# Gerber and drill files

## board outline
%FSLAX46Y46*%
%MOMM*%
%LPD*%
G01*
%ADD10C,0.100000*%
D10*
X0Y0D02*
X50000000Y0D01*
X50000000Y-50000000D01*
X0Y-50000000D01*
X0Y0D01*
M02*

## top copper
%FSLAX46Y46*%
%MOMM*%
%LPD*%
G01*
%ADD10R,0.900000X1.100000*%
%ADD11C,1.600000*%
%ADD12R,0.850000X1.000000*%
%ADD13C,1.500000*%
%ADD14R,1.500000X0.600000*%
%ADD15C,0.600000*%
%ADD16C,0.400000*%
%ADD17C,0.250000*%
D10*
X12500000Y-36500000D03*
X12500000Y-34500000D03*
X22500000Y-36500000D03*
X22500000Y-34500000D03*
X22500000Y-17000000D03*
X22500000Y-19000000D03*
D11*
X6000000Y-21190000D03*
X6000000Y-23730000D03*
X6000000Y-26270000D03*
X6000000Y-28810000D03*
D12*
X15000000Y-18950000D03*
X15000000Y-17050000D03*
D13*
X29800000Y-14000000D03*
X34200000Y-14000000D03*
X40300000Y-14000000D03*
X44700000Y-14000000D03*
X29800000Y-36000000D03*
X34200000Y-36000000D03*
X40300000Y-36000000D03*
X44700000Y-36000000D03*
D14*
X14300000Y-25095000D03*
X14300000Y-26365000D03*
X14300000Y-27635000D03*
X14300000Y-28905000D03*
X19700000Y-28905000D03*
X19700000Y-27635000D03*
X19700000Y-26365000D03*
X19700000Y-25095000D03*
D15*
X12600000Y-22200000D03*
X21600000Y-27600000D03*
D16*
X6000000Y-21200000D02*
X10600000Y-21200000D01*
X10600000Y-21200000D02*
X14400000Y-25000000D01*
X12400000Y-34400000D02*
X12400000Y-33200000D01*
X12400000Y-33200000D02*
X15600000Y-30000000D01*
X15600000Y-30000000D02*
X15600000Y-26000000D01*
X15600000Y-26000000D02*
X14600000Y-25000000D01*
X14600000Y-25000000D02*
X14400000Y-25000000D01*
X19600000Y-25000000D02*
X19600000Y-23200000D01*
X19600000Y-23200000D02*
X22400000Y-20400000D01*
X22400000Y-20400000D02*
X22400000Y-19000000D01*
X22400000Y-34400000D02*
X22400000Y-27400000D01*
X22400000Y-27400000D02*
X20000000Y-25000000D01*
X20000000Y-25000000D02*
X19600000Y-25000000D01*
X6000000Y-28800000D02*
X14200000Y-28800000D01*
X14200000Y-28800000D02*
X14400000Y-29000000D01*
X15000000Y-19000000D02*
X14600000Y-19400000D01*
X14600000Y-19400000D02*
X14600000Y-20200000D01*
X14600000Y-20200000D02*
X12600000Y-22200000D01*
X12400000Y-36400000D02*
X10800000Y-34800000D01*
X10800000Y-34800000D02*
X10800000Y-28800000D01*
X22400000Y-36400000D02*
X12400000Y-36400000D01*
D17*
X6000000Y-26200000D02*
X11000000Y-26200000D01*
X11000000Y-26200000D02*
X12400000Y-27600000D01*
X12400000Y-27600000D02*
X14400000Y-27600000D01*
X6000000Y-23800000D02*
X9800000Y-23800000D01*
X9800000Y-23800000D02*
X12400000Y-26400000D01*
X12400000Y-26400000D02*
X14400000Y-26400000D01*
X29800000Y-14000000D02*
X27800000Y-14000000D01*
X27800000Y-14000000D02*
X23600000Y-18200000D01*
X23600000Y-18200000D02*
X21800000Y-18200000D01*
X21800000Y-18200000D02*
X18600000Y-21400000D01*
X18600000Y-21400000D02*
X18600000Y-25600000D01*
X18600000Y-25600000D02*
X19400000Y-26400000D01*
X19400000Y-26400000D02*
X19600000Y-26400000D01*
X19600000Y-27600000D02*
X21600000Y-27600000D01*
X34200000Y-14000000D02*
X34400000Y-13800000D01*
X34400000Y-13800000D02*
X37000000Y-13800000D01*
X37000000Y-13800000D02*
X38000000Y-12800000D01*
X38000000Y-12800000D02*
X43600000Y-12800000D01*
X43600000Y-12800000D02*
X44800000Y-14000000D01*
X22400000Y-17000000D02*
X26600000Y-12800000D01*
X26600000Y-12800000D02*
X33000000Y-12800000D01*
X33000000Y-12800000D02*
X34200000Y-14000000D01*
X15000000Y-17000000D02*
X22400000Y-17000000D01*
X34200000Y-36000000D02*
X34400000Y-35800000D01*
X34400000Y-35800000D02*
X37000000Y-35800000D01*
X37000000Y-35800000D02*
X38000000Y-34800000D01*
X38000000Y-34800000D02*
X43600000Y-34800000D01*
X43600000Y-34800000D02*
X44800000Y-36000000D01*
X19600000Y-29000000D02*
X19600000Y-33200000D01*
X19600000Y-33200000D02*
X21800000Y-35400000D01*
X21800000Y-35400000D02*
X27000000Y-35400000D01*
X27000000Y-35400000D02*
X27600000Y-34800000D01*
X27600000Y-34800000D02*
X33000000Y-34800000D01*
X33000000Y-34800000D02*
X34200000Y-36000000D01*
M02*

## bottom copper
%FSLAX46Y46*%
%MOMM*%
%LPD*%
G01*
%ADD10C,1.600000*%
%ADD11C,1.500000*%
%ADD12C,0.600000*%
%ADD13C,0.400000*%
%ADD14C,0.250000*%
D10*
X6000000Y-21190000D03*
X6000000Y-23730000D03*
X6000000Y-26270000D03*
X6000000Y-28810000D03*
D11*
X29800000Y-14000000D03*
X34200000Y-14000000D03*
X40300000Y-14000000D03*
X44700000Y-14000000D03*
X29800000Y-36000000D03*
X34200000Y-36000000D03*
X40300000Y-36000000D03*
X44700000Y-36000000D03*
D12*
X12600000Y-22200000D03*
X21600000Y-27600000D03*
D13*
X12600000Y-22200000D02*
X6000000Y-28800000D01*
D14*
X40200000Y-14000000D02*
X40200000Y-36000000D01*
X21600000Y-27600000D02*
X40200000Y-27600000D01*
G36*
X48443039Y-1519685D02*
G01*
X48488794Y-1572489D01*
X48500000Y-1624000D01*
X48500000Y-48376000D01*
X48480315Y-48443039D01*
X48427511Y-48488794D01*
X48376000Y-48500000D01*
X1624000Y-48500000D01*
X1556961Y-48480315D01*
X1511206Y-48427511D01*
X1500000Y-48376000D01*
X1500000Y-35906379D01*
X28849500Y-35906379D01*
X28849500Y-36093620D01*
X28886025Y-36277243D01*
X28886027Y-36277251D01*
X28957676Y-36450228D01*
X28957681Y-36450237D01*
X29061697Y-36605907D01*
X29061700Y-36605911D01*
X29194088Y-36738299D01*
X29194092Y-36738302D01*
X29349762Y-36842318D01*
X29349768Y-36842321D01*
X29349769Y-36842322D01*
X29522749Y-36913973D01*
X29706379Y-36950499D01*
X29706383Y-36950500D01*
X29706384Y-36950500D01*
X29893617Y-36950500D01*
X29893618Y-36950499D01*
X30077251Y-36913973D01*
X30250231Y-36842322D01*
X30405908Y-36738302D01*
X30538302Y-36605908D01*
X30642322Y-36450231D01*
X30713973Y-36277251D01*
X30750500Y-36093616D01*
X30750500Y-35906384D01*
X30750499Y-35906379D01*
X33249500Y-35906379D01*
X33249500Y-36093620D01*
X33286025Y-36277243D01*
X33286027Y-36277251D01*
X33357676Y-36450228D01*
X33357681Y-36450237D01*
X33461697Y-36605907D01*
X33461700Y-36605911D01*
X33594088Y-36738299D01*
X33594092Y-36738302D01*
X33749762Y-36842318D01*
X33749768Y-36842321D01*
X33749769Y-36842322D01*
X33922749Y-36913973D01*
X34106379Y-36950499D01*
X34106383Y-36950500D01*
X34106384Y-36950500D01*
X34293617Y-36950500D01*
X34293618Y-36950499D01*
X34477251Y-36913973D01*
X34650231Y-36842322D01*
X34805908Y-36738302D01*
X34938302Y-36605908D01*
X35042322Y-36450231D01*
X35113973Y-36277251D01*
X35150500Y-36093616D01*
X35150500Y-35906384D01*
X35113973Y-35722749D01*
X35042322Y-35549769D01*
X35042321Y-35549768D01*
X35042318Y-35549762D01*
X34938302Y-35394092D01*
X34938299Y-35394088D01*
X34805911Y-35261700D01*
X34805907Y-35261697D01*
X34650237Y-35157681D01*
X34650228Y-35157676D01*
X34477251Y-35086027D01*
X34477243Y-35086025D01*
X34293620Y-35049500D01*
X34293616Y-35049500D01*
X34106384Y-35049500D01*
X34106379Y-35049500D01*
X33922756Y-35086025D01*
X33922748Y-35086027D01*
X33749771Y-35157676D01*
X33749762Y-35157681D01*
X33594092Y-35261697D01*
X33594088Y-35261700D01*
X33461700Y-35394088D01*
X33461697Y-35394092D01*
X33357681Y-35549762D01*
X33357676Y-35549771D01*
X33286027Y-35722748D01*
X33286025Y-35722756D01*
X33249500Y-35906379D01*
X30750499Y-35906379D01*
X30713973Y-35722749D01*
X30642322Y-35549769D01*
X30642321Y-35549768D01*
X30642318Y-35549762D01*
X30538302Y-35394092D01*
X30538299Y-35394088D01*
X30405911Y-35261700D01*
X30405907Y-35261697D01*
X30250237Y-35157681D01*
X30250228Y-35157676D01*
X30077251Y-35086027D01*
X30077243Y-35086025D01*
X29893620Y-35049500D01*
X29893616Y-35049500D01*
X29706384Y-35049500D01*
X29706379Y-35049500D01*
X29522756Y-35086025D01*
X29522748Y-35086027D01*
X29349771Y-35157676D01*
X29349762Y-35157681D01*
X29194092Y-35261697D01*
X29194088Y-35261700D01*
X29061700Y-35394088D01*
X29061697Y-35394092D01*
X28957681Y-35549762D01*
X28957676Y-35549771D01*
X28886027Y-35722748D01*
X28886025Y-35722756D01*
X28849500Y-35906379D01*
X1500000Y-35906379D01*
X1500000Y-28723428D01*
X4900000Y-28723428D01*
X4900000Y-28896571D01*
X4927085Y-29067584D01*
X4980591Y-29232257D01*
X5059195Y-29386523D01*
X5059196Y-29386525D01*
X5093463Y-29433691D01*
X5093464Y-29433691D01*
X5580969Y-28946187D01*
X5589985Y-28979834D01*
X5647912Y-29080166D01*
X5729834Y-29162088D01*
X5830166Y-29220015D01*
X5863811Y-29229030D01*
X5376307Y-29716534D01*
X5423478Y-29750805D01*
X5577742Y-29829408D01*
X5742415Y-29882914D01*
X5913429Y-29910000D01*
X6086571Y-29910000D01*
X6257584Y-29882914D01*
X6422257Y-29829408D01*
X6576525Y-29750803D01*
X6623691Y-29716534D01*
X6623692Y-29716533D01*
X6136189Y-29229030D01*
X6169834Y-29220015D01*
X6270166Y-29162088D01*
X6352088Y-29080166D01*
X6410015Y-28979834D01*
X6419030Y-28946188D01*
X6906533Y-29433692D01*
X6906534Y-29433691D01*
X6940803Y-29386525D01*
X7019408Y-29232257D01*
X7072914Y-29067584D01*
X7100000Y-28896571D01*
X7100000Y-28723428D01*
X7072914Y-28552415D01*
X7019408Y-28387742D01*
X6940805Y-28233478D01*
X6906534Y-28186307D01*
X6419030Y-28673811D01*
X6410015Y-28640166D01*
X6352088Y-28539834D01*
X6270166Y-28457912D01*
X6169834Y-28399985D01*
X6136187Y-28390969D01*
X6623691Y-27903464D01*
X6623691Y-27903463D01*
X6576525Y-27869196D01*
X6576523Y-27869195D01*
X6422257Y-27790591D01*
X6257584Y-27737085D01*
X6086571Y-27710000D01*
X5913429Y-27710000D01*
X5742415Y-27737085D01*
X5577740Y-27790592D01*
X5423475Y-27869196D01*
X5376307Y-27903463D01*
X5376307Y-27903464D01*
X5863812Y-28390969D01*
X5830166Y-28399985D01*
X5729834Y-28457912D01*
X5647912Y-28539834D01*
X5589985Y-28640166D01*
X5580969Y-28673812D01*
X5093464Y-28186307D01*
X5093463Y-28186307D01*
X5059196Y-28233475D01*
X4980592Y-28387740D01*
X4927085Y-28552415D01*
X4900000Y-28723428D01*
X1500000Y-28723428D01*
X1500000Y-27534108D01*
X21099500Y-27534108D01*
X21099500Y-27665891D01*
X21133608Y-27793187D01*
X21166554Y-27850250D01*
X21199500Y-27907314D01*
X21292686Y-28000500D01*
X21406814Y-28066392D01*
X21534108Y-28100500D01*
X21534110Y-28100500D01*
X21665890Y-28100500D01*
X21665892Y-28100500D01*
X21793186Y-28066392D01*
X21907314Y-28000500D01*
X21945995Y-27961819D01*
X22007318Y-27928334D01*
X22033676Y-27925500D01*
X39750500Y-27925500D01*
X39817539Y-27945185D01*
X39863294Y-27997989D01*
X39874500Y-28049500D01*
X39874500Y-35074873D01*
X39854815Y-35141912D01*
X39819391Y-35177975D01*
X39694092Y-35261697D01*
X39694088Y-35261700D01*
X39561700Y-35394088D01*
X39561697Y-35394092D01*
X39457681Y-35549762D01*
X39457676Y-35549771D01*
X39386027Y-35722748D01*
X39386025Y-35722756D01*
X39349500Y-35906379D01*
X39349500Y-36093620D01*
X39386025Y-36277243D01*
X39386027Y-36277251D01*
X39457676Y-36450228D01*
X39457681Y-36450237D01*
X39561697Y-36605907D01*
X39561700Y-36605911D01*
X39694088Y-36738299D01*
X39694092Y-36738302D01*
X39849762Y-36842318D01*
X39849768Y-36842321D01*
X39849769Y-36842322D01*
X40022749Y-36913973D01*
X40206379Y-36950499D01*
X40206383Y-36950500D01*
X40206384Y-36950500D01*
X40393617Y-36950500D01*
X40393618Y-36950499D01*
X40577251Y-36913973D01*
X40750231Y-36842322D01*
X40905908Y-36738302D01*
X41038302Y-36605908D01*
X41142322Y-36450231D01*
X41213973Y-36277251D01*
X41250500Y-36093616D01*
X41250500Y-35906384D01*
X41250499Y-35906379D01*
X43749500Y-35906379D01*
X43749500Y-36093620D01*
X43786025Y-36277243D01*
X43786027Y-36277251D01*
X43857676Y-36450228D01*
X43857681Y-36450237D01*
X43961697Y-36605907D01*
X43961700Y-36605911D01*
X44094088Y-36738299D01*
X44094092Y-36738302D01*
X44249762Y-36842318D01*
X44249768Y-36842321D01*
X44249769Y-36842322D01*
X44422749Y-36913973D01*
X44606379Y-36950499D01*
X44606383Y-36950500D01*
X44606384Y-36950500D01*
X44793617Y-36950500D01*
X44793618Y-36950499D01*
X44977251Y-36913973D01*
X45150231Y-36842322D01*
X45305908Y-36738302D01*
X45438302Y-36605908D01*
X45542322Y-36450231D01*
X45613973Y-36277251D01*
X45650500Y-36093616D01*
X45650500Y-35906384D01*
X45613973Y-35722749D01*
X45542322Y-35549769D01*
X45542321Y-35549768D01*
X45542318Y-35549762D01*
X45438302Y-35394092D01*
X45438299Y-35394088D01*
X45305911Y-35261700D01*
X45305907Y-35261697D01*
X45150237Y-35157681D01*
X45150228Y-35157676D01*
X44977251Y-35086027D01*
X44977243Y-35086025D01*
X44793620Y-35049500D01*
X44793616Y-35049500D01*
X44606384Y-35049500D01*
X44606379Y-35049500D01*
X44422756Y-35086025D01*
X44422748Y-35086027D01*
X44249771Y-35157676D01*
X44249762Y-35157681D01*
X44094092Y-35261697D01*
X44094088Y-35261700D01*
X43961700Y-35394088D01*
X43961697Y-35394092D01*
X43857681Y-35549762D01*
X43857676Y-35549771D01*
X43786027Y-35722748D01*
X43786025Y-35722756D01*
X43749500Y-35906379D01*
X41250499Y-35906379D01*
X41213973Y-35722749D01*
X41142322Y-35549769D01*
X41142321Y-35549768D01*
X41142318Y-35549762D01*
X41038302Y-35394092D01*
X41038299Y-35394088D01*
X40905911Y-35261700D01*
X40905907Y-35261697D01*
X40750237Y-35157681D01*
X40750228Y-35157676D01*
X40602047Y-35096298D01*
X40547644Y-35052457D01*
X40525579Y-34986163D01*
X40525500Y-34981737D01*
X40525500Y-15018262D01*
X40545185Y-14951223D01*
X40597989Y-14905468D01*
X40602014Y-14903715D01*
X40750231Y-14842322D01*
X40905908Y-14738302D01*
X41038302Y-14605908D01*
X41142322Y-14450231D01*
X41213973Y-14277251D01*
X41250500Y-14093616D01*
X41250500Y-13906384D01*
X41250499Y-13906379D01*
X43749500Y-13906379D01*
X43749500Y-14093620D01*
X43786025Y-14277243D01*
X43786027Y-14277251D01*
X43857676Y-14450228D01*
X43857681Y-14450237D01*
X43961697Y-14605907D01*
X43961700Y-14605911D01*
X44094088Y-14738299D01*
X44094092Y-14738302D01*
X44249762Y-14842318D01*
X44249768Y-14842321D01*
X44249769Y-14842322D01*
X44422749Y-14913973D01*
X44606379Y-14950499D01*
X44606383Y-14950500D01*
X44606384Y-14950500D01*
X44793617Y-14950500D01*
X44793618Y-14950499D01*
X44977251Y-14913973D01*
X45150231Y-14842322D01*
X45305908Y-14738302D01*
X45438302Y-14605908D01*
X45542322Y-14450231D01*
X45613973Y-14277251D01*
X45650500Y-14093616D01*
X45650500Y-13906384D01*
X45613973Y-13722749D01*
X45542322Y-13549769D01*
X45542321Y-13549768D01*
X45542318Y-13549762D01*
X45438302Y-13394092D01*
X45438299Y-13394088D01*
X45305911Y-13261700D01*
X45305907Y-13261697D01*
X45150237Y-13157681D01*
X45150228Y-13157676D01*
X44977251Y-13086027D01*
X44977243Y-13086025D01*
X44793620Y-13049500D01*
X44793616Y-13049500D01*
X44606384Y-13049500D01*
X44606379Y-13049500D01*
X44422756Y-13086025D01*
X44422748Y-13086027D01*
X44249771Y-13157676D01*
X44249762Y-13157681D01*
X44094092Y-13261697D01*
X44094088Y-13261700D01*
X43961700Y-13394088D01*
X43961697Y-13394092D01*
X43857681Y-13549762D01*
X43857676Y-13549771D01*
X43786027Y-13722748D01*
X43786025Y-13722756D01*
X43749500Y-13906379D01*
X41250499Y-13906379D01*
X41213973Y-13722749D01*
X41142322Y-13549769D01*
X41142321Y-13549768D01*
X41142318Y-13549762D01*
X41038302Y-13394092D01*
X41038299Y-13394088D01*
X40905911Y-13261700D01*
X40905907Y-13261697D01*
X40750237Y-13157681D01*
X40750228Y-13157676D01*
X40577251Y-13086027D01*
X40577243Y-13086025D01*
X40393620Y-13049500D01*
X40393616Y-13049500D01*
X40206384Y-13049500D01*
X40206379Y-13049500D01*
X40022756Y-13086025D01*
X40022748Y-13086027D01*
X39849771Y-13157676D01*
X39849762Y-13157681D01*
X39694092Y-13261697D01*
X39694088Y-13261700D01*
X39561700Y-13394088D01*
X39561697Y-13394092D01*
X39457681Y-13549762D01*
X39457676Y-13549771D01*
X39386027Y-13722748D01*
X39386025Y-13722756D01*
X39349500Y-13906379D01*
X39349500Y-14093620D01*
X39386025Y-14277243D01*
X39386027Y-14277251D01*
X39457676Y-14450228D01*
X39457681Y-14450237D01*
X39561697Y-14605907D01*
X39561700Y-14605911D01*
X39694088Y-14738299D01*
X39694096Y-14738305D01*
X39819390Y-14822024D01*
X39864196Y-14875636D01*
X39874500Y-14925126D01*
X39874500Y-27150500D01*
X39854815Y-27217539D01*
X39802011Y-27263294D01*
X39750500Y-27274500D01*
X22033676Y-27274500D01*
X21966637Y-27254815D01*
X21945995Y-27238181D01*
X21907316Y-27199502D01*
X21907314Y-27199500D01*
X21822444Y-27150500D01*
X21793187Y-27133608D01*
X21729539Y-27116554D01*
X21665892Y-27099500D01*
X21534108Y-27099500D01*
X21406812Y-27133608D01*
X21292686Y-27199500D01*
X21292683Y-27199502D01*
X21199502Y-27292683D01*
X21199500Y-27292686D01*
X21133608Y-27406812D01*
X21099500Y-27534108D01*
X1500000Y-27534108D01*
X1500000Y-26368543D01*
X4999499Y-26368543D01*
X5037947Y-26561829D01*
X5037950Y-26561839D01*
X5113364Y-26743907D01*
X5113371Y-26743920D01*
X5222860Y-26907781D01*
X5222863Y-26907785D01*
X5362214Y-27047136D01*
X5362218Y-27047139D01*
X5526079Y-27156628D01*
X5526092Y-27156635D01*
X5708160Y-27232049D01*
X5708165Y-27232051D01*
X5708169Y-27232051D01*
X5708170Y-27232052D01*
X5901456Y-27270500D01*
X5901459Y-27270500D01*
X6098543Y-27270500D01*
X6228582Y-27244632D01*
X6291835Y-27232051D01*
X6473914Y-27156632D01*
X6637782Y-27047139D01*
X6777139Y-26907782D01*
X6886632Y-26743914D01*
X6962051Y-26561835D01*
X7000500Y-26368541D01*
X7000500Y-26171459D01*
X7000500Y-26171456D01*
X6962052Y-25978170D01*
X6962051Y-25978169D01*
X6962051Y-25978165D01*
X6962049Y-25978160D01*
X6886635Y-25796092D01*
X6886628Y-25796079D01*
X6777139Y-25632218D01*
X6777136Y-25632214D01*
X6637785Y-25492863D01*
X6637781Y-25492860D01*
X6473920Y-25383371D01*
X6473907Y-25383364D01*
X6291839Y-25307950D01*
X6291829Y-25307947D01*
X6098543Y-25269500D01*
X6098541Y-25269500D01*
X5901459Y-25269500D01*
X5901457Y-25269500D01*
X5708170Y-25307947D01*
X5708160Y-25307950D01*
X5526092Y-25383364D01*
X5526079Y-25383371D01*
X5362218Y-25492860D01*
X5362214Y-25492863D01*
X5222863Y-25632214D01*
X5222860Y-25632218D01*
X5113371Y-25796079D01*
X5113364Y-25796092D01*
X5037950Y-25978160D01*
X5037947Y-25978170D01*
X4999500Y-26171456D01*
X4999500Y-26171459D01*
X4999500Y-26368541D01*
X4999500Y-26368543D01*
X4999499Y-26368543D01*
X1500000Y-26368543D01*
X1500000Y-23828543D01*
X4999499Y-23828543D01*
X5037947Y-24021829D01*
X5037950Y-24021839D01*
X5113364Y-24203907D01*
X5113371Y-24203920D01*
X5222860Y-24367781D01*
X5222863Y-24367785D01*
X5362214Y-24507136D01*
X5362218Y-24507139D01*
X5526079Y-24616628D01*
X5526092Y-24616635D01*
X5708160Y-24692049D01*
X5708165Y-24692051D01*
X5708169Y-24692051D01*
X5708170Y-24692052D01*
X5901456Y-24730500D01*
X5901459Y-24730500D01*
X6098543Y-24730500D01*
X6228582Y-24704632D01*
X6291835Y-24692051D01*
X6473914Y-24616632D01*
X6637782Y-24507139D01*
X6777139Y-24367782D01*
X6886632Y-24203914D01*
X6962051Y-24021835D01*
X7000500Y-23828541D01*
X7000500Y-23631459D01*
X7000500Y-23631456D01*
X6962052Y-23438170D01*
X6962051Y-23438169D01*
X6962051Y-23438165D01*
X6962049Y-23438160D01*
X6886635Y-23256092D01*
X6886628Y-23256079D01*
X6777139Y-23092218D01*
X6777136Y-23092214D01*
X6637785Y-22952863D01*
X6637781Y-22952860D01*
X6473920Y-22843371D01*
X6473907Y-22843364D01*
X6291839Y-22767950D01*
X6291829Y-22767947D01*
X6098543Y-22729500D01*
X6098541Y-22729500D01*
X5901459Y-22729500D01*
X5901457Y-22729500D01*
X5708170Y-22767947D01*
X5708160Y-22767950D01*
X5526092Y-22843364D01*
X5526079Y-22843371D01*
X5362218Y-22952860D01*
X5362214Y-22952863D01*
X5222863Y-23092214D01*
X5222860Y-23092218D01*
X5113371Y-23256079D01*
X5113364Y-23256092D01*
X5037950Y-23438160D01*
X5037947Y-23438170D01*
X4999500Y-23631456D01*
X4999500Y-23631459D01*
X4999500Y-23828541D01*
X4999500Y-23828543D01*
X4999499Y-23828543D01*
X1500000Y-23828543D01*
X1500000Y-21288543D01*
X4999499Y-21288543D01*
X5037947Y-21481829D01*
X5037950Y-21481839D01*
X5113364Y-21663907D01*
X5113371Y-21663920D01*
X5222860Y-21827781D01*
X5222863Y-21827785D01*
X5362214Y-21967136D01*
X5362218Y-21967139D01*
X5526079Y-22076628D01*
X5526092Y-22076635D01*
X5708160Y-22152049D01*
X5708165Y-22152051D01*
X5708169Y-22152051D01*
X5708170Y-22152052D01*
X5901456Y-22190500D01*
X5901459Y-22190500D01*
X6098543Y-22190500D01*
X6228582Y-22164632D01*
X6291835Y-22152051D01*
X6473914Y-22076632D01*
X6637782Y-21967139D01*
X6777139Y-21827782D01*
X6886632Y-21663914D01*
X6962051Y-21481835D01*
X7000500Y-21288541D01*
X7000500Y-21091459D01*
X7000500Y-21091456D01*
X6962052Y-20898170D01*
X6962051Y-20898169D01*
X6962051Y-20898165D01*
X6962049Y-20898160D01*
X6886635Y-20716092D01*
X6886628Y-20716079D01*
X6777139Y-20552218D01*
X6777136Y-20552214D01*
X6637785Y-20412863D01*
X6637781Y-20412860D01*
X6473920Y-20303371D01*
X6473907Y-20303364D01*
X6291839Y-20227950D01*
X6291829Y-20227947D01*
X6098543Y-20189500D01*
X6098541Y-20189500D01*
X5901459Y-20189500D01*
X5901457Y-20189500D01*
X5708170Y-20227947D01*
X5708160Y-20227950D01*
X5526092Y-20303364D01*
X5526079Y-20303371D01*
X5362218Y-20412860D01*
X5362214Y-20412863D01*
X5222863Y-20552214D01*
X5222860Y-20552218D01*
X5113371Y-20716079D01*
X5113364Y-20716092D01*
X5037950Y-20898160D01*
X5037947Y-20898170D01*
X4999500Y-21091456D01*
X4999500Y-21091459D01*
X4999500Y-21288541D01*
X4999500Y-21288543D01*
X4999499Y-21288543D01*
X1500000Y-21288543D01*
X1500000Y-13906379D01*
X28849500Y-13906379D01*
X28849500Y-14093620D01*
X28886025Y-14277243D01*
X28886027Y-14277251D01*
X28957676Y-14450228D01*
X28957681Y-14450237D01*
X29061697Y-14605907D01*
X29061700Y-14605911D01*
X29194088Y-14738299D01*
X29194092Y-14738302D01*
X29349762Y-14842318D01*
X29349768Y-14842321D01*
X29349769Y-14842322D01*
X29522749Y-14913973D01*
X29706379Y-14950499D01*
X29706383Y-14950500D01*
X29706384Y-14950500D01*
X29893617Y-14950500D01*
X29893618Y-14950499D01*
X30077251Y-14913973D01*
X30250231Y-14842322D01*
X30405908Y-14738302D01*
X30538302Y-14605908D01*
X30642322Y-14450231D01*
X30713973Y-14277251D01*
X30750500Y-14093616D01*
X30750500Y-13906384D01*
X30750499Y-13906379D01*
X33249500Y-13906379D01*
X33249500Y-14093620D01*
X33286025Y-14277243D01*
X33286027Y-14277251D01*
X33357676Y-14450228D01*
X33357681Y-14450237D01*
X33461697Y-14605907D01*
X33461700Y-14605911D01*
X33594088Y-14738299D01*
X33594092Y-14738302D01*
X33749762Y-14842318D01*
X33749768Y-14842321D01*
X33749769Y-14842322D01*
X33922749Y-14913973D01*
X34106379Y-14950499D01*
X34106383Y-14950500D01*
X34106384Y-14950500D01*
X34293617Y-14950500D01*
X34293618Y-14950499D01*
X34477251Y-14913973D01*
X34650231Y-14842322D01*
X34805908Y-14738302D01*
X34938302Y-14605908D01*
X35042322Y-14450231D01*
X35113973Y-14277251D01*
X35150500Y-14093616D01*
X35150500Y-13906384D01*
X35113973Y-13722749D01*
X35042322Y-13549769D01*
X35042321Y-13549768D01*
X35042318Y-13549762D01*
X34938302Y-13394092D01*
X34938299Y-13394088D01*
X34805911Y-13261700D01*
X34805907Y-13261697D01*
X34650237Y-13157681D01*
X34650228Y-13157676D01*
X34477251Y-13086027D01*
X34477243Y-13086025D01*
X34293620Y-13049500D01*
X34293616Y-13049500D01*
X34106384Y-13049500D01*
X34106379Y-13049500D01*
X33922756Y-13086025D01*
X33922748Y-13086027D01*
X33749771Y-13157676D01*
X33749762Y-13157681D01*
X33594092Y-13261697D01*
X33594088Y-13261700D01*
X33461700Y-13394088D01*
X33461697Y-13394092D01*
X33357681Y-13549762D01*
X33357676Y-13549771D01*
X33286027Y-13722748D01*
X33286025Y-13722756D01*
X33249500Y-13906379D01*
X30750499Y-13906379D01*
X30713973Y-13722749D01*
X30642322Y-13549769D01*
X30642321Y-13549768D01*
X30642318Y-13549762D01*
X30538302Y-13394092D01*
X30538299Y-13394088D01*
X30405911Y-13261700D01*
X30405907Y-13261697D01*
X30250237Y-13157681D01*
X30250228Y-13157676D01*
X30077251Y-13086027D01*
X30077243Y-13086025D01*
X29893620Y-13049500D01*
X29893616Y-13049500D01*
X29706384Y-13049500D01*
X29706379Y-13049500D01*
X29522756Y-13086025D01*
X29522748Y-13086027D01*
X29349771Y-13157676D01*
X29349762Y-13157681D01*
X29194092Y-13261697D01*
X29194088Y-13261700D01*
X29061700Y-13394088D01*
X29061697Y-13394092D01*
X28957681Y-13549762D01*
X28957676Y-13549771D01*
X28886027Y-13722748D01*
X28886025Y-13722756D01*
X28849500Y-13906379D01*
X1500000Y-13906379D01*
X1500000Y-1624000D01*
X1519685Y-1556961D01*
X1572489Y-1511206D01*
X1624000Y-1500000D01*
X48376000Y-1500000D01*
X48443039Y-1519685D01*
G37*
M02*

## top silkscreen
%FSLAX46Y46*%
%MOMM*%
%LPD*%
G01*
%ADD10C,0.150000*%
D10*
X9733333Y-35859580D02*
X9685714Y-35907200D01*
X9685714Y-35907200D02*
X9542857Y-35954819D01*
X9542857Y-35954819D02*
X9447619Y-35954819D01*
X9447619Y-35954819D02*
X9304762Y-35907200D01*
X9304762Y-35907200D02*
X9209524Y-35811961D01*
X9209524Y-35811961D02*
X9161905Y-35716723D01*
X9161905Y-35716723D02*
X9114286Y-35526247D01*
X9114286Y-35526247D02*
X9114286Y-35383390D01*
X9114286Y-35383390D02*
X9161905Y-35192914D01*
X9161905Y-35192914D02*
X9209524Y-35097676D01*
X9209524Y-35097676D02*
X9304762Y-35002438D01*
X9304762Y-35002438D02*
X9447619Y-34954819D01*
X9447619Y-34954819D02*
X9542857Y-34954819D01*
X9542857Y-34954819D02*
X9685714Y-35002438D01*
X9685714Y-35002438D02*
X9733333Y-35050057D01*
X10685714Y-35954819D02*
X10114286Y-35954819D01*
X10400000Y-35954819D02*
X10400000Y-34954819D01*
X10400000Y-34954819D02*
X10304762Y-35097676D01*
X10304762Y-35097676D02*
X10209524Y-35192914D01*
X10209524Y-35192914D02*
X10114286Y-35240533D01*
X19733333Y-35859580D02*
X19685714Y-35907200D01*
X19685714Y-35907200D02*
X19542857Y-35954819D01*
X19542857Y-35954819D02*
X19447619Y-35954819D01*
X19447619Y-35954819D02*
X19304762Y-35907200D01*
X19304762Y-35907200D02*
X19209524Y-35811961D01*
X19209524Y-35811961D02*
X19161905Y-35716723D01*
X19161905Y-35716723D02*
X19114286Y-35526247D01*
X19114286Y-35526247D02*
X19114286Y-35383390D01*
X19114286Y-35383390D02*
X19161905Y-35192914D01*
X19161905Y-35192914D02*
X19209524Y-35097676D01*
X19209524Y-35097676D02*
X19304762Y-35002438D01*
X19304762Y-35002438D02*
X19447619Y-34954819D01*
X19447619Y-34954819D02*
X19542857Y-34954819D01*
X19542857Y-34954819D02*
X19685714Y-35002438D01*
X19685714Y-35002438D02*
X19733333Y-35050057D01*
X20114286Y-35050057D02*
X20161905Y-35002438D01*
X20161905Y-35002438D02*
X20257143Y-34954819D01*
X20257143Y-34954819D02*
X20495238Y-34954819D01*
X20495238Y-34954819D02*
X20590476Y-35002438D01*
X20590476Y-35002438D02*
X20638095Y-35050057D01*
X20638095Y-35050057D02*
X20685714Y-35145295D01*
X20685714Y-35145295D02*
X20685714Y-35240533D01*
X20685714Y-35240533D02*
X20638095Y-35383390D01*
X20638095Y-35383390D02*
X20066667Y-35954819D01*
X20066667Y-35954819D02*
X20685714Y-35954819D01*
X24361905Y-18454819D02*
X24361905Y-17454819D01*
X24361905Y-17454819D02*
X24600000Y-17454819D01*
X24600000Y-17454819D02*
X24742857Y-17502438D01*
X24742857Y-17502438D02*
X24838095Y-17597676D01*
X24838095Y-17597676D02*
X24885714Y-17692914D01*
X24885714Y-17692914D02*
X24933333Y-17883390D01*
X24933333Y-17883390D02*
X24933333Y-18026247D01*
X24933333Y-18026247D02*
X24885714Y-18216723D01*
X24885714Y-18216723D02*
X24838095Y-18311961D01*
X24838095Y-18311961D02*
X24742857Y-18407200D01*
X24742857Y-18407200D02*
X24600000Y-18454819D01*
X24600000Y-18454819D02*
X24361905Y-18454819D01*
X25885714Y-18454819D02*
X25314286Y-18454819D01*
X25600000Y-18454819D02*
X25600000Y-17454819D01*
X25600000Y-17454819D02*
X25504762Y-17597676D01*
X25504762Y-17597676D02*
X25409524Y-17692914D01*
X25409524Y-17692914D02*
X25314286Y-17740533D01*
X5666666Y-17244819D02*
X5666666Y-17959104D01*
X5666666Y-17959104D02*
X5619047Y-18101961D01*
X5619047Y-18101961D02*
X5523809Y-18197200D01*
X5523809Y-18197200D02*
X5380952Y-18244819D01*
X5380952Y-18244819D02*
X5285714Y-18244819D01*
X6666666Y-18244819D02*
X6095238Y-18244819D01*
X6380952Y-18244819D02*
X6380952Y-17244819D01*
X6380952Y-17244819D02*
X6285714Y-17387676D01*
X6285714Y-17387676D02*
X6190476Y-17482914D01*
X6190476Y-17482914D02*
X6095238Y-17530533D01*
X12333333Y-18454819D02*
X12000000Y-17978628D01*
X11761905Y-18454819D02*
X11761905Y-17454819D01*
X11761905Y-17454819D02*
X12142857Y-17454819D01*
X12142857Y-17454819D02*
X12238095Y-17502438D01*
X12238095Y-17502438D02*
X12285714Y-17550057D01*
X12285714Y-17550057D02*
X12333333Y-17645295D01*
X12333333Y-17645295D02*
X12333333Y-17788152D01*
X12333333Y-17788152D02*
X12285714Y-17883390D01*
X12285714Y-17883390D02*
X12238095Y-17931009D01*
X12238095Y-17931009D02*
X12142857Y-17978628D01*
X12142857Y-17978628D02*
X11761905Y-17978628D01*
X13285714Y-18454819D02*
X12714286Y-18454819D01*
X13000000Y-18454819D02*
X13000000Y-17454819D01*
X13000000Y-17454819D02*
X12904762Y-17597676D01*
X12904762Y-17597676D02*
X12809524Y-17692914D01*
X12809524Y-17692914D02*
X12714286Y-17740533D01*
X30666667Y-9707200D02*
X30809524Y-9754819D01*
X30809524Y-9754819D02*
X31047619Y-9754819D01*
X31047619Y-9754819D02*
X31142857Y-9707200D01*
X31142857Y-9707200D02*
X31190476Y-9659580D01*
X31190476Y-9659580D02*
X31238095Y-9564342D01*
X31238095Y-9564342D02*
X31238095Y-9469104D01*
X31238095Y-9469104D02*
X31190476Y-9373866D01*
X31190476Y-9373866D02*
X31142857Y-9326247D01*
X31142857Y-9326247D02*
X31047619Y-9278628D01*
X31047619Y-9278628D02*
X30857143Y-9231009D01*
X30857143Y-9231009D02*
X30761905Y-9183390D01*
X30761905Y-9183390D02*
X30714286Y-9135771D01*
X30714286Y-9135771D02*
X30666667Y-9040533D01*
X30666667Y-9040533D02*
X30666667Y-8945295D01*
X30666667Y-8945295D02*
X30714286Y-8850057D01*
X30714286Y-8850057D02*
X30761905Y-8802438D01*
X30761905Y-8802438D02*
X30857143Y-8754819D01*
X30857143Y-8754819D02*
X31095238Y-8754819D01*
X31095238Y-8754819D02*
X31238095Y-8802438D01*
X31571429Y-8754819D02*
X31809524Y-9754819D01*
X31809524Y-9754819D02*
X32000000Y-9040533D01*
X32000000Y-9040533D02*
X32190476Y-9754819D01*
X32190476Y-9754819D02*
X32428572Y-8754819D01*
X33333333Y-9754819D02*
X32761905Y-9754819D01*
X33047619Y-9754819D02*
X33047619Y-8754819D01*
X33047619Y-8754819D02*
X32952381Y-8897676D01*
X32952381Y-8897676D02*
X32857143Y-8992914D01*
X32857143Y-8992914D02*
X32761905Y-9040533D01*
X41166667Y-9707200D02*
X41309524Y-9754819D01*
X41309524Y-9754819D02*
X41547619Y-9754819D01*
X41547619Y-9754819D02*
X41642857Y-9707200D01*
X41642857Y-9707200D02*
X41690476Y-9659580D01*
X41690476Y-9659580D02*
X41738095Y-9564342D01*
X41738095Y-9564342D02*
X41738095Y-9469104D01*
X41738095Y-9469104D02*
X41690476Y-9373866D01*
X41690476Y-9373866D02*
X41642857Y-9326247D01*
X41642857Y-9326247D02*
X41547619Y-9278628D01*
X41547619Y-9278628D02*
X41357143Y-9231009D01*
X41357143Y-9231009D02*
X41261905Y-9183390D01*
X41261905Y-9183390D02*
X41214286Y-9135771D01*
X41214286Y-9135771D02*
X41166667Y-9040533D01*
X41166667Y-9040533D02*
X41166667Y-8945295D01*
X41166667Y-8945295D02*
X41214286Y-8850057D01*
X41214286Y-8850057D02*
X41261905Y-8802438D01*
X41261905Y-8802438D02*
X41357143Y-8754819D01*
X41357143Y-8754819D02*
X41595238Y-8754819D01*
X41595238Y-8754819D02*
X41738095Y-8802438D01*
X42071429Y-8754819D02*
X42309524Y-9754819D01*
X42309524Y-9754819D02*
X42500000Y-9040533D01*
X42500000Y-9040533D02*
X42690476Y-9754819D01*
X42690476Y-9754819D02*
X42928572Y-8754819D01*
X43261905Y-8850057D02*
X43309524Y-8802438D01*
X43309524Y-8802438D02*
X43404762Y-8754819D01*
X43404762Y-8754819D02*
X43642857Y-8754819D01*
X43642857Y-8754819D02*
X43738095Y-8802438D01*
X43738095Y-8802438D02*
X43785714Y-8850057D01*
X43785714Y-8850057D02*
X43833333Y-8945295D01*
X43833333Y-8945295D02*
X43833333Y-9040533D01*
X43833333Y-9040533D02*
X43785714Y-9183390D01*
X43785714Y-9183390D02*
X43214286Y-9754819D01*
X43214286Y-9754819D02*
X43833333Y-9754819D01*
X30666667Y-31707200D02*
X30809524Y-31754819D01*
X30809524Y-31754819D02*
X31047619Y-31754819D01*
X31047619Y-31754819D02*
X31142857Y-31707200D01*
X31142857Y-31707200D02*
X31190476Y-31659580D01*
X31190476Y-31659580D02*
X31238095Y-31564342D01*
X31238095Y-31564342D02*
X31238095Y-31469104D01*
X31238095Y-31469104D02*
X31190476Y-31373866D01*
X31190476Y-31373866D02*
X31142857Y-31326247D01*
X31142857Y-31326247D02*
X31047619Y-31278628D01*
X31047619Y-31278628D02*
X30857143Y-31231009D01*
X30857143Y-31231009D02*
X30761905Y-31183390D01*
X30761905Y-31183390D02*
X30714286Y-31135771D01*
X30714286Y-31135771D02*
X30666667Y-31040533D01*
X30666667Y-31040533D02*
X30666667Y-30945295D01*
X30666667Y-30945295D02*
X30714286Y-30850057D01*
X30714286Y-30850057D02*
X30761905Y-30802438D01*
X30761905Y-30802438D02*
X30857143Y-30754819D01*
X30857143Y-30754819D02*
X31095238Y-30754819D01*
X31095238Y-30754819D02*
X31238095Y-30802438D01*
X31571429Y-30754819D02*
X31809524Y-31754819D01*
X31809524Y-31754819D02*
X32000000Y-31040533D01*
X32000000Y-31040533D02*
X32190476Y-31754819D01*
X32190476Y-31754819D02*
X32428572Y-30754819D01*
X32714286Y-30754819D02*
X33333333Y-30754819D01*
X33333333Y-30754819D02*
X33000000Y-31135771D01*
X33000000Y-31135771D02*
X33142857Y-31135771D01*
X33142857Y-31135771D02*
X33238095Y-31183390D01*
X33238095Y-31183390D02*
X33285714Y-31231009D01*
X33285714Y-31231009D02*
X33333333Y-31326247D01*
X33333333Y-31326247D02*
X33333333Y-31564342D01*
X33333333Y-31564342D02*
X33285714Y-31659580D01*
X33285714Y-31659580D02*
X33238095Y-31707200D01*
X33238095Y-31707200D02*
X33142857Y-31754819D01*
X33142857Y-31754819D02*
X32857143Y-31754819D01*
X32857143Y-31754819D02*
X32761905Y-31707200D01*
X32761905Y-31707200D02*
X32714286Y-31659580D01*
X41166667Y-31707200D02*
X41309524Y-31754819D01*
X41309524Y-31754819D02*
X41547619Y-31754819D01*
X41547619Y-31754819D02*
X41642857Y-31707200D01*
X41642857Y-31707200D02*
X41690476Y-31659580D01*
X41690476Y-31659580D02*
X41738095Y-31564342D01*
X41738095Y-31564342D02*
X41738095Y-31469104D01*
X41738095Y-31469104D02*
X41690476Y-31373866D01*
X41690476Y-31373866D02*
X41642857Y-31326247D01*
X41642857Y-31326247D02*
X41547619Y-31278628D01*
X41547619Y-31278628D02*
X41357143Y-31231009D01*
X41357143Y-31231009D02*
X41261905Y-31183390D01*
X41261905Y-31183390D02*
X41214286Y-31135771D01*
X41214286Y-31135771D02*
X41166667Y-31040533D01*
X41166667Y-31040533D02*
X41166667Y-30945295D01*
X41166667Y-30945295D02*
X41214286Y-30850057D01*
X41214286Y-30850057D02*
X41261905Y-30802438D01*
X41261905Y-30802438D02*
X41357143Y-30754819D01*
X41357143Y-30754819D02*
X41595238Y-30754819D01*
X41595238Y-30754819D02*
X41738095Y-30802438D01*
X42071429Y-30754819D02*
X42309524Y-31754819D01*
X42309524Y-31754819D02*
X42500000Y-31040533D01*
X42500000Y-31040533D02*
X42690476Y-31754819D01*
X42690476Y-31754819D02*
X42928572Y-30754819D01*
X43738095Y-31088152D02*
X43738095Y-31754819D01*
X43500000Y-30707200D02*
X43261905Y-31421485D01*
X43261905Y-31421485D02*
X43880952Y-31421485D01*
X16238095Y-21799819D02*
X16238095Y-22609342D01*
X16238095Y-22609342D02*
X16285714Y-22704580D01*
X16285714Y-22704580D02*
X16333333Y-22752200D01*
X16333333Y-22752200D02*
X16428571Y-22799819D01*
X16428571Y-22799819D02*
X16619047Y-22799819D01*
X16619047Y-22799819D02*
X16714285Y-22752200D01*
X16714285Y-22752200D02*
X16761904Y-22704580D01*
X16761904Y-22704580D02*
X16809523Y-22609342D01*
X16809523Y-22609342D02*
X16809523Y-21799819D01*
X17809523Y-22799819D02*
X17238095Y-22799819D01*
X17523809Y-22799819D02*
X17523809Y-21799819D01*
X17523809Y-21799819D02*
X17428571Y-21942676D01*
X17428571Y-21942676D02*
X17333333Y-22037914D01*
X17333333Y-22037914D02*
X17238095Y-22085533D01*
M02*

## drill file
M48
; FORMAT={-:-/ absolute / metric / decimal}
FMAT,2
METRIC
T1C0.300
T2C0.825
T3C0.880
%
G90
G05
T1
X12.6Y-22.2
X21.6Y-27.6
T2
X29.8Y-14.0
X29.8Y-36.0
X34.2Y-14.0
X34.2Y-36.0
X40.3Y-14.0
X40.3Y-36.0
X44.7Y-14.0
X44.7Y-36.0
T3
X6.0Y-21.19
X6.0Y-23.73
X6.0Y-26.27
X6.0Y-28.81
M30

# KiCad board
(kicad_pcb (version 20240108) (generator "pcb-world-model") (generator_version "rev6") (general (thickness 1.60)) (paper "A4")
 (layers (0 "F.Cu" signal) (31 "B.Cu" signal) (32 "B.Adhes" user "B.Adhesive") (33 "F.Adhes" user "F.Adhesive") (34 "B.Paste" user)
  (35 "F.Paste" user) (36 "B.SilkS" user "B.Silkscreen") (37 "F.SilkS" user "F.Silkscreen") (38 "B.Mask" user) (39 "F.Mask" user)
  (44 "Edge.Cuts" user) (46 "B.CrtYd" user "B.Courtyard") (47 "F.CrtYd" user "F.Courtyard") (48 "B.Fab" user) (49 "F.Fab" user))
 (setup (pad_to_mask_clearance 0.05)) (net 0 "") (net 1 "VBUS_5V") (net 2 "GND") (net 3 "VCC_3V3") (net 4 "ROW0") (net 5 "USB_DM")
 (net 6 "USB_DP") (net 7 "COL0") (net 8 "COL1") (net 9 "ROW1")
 (gr_rect (start 0.0 0.0) (end 50.0000 50.0000) (stroke (width 0.1) (type default)) (fill none) (layer "Edge.Cuts"))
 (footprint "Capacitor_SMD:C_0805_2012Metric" (layer "F.Cu") (at 12.5000 35.5000 90)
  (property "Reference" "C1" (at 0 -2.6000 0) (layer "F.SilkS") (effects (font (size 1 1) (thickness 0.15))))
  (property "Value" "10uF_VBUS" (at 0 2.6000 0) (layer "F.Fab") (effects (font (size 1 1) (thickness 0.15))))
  (pad "1" smd rect (at -1.0000 0.0000) (size 0.9000 1.1000) (layers "F.Cu" "F.Paste" "F.Mask") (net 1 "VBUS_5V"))
  (pad "2" smd rect (at 1.0000 0.0000) (size 0.9000 1.1000) (layers "F.Cu" "F.Paste" "F.Mask") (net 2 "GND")))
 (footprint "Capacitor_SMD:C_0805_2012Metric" (layer "F.Cu") (at 22.5000 35.5000 90)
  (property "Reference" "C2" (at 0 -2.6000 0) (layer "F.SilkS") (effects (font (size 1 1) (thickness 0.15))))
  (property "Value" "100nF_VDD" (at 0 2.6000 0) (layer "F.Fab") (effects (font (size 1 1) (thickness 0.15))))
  (pad "1" smd rect (at -1.0000 0.0000) (size 0.9000 1.1000) (layers "F.Cu" "F.Paste" "F.Mask") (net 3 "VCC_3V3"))
  (pad "2" smd rect (at 1.0000 0.0000) (size 0.9000 1.1000) (layers "F.Cu" "F.Paste" "F.Mask") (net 2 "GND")))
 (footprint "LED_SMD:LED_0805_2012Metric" (layer "F.Cu") (at 22.5000 18.0000 270)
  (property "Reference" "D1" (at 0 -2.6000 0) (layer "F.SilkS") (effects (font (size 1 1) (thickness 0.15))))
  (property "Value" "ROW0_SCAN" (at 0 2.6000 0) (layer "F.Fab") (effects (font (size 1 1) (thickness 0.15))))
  (pad "1" smd rect (at -1.0000 0.0000) (size 0.9000 1.1000) (layers "F.Cu" "F.Paste" "F.Mask") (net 3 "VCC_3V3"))
  (pad "2" smd rect (at 1.0000 0.0000) (size 0.9000 1.1000) (layers "F.Cu" "F.Paste" "F.Mask") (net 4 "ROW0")))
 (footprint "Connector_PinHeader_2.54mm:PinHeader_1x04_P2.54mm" (layer "F.Cu") (at 6.0000 25.0000 0) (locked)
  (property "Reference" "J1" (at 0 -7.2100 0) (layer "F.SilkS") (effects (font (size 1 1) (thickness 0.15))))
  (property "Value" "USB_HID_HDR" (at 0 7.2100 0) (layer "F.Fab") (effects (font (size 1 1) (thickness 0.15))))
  (pad "1" thru_hole circle (at 0.0000 -3.8100) (size 1.6000 1.6000) (drill 0.8800) (layers "*.Cu" "*.Mask") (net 1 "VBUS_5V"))
  (pad "2" thru_hole circle (at 0.0000 -1.2700) (size 1.6000 1.6000) (drill 0.8800) (layers "*.Cu" "*.Mask") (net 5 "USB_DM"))
  (pad "3" thru_hole circle (at 0.0000 1.2700) (size 1.6000 1.6000) (drill 0.8800) (layers "*.Cu" "*.Mask") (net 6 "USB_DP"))
  (pad "4" thru_hole circle (at 0.0000 3.8100) (size 1.6000 1.6000) (drill 0.8800) (layers "*.Cu" "*.Mask") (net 2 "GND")))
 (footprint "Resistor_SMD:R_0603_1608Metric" (layer "F.Cu") (at 15.0000 18.0000 90)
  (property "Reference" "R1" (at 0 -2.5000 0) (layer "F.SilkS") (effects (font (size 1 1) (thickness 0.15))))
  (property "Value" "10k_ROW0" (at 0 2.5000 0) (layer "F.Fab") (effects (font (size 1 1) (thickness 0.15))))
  (pad "1" smd rect (at -0.9500 0.0000) (size 0.8500 1.0000) (layers "F.Cu" "F.Paste" "F.Mask") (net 4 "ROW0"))
  (pad "2" smd rect (at 0.9500 0.0000) (size 0.8500 1.0000) (layers "F.Cu" "F.Paste" "F.Mask") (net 2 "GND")))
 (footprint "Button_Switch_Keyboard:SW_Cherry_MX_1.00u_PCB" (layer "F.Cu") (at 32.0000 14.0000 0) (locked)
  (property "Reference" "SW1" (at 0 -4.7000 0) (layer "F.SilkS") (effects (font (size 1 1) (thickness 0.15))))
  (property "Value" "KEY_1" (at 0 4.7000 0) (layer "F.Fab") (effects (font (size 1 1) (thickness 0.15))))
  (pad "1" thru_hole circle (at -2.2000 0.0000) (size 1.5000 1.5000) (drill 0.8250) (layers "*.Cu" "*.Mask") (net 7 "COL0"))
  (pad "2" thru_hole circle (at 2.2000 0.0000) (size 1.5000 1.5000) (drill 0.8250) (layers "*.Cu" "*.Mask") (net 4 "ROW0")))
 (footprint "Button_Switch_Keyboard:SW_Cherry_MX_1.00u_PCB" (layer "F.Cu") (at 42.5000 14.0000 0) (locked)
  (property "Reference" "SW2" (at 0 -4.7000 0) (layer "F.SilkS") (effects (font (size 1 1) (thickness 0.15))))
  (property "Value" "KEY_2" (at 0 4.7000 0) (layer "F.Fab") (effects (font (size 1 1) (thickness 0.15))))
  (pad "1" thru_hole circle (at -2.2000 0.0000) (size 1.5000 1.5000) (drill 0.8250) (layers "*.Cu" "*.Mask") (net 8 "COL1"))
  (pad "2" thru_hole circle (at 2.2000 0.0000) (size 1.5000 1.5000) (drill 0.8250) (layers "*.Cu" "*.Mask") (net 4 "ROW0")))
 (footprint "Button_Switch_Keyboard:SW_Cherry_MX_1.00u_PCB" (layer "F.Cu") (at 32.0000 36.0000 0) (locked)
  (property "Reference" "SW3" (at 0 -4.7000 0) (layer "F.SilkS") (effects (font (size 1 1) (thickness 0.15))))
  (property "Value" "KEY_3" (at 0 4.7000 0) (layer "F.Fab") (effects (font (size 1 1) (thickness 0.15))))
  (pad "1" thru_hole circle (at -2.2000 0.0000) (size 1.5000 1.5000) (drill 0.8250) (layers "*.Cu" "*.Mask") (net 7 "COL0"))
  (pad "2" thru_hole circle (at 2.2000 0.0000) (size 1.5000 1.5000) (drill 0.8250) (layers "*.Cu" "*.Mask") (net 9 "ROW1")))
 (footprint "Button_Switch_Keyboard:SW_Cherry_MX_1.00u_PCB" (layer "F.Cu") (at 42.5000 36.0000 0) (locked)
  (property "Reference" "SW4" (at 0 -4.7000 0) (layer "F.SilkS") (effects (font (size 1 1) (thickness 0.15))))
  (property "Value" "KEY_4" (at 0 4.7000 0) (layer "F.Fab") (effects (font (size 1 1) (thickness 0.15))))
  (pad "1" thru_hole circle (at -2.2000 0.0000) (size 1.5000 1.5000) (drill 0.8250) (layers "*.Cu" "*.Mask") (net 8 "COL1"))
  (pad "2" thru_hole circle (at 2.2000 0.0000) (size 1.5000 1.5000) (drill 0.8250) (layers "*.Cu" "*.Mask") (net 9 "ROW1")))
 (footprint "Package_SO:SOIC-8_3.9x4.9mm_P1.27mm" (layer "F.Cu") (at 17.0000 27.0000 0)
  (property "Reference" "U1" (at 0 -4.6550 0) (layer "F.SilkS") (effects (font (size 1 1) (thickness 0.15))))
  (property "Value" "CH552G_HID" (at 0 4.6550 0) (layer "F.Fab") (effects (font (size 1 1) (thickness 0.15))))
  (pad "1" smd rect (at -2.7000 -1.9050) (size 1.5000 0.6000) (layers "F.Cu" "F.Paste" "F.Mask") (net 1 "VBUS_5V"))
  (pad "2" smd rect (at -2.7000 -0.6350) (size 1.5000 0.6000) (layers "F.Cu" "F.Paste" "F.Mask") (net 5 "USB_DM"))
  (pad "3" smd rect (at -2.7000 0.6350) (size 1.5000 0.6000) (layers "F.Cu" "F.Paste" "F.Mask") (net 6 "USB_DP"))
  (pad "4" smd rect (at -2.7000 1.9050) (size 1.5000 0.6000) (layers "F.Cu" "F.Paste" "F.Mask") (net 2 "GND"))
  (pad "5" smd rect (at 2.7000 1.9050) (size 1.5000 0.6000) (layers "F.Cu" "F.Paste" "F.Mask") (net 9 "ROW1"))
  (pad "6" smd rect (at 2.7000 0.6350) (size 1.5000 0.6000) (layers "F.Cu" "F.Paste" "F.Mask") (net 8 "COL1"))
  (pad "7" smd rect (at 2.7000 -0.6350) (size 1.5000 0.6000) (layers "F.Cu" "F.Paste" "F.Mask") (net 7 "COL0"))
  (pad "8" smd rect (at 2.7000 -1.9050) (size 1.5000 0.6000) (layers "F.Cu" "F.Paste" "F.Mask") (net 3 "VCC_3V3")))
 (segment (start 6.0000 21.2000) (end 10.6000 21.2000) (width 0.4000) (layer "F.Cu") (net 1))
 (segment (start 10.6000 21.2000) (end 14.4000 25.0000) (width 0.4000) (layer "F.Cu") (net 1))
 (segment (start 12.4000 34.4000) (end 12.4000 33.2000) (width 0.4000) (layer "F.Cu") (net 1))
 (segment (start 12.4000 33.2000) (end 15.6000 30.0000) (width 0.4000) (layer "F.Cu") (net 1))
 (segment (start 15.6000 30.0000) (end 15.6000 26.0000) (width 0.4000) (layer "F.Cu") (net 1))
 (segment (start 15.6000 26.0000) (end 14.6000 25.0000) (width 0.4000) (layer "F.Cu") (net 1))
 (segment (start 14.6000 25.0000) (end 14.4000 25.0000) (width 0.4000) (layer "F.Cu") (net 1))
 (segment (start 19.6000 25.0000) (end 19.6000 23.2000) (width 0.4000) (layer "F.Cu") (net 3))
 (segment (start 19.6000 23.2000) (end 22.4000 20.4000) (width 0.4000) (layer "F.Cu") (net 3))
 (segment (start 22.4000 20.4000) (end 22.4000 19.0000) (width 0.4000) (layer "F.Cu") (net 3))
 (segment (start 22.4000 34.4000) (end 22.4000 27.4000) (width 0.4000) (layer "F.Cu") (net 3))
 (segment (start 22.4000 27.4000) (end 20.0000 25.0000) (width 0.4000) (layer "F.Cu") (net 3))
 (segment (start 20.0000 25.0000) (end 19.6000 25.0000) (width 0.4000) (layer "F.Cu") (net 3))
 (segment (start 6.0000 28.8000) (end 14.2000 28.8000) (width 0.4000) (layer "F.Cu") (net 2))
 (segment (start 14.2000 28.8000) (end 14.4000 29.0000) (width 0.4000) (layer "F.Cu") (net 2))
 (segment (start 15.0000 19.0000) (end 14.6000 19.4000) (width 0.4000) (layer "F.Cu") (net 2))
 (segment (start 14.6000 19.4000) (end 14.6000 20.2000) (width 0.4000) (layer "F.Cu") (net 2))
 (segment (start 14.6000 20.2000) (end 12.6000 22.2000) (width 0.4000) (layer "F.Cu") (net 2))
 (segment (start 12.6000 22.2000) (end 6.0000 28.8000) (width 0.4000) (layer "B.Cu") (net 2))
 (segment (start 12.4000 36.4000) (end 10.8000 34.8000) (width 0.4000) (layer "F.Cu") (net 2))
 (segment (start 10.8000 34.8000) (end 10.8000 28.8000) (width 0.4000) (layer "F.Cu") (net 2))
 (segment (start 22.4000 36.4000) (end 12.4000 36.4000) (width 0.4000) (layer "F.Cu") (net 2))
 (segment (start 6.0000 26.2000) (end 11.0000 26.2000) (width 0.2500) (layer "F.Cu") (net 6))
 (segment (start 11.0000 26.2000) (end 12.4000 27.6000) (width 0.2500) (layer "F.Cu") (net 6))
 (segment (start 12.4000 27.6000) (end 14.4000 27.6000) (width 0.2500) (layer "F.Cu") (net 6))
 (segment (start 6.0000 23.8000) (end 9.8000 23.8000) (width 0.2500) (layer "F.Cu") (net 5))
 (segment (start 9.8000 23.8000) (end 12.4000 26.4000) (width 0.2500) (layer "F.Cu") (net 5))
 (segment (start 12.4000 26.4000) (end 14.4000 26.4000) (width 0.2500) (layer "F.Cu") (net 5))
 (segment (start 29.8000 14.0000) (end 27.8000 14.0000) (width 0.2500) (layer "F.Cu") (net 7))
 (segment (start 27.8000 14.0000) (end 23.6000 18.2000) (width 0.2500) (layer "F.Cu") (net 7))
 (segment (start 23.6000 18.2000) (end 21.8000 18.2000) (width 0.2500) (layer "F.Cu") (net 7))
 (segment (start 21.8000 18.2000) (end 18.6000 21.4000) (width 0.2500) (layer "F.Cu") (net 7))
 (segment (start 18.6000 21.4000) (end 18.6000 25.6000) (width 0.2500) (layer "F.Cu") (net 7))
 (segment (start 18.6000 25.6000) (end 19.4000 26.4000) (width 0.2500) (layer "F.Cu") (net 7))
 (segment (start 19.4000 26.4000) (end 19.6000 26.4000) (width 0.2500) (layer "F.Cu") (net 7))
 (segment (start 40.2000 14.0000) (end 40.2000 36.0000) (width 0.2500) (layer "B.Cu") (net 8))
 (segment (start 19.6000 27.6000) (end 21.6000 27.6000) (width 0.2500) (layer "F.Cu") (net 8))
 (segment (start 21.6000 27.6000) (end 40.2000 27.6000) (width 0.2500) (layer "B.Cu") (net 8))
 (segment (start 34.2000 14.0000) (end 34.4000 13.8000) (width 0.2500) (layer "F.Cu") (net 4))
 (segment (start 34.4000 13.8000) (end 37.0000 13.8000) (width 0.2500) (layer "F.Cu") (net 4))
 (segment (start 37.0000 13.8000) (end 38.0000 12.8000) (width 0.2500) (layer "F.Cu") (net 4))
 (segment (start 38.0000 12.8000) (end 43.6000 12.8000) (width 0.2500) (layer "F.Cu") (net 4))
 (segment (start 43.6000 12.8000) (end 44.8000 14.0000) (width 0.2500) (layer "F.Cu") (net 4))
 (segment (start 22.4000 17.0000) (end 26.6000 12.8000) (width 0.2500) (layer "F.Cu") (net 4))
 (segment (start 26.6000 12.8000) (end 33.0000 12.8000) (width 0.2500) (layer "F.Cu") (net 4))
 (segment (start 33.0000 12.8000) (end 34.2000 14.0000) (width 0.2500) (layer "F.Cu") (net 4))
 (segment (start 15.0000 17.0000) (end 22.4000 17.0000) (width 0.2500) (layer "F.Cu") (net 4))
 (segment (start 34.2000 36.0000) (end 34.4000 35.8000) (width 0.2500) (layer "F.Cu") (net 9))
 (segment (start 34.4000 35.8000) (end 37.0000 35.8000) (width 0.2500) (layer "F.Cu") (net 9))
 (segment (start 37.0000 35.8000) (end 38.0000 34.8000) (width 0.2500) (layer "F.Cu") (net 9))
 (segment (start 38.0000 34.8000) (end 43.6000 34.8000) (width 0.2500) (layer "F.Cu") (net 9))
 (segment (start 43.6000 34.8000) (end 44.8000 36.0000) (width 0.2500) (layer "F.Cu") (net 9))
 (segment (start 19.6000 29.0000) (end 19.6000 33.2000) (width 0.2500) (layer "F.Cu") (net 9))
 (segment (start 19.6000 33.2000) (end 21.8000 35.4000) (width 0.2500) (layer "F.Cu") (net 9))
 (segment (start 21.8000 35.4000) (end 27.0000 35.4000) (width 0.2500) (layer "F.Cu") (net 9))
 (segment (start 27.0000 35.4000) (end 27.6000 34.8000) (width 0.2500) (layer "F.Cu") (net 9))
 (segment (start 27.6000 34.8000) (end 33.0000 34.8000) (width 0.2500) (layer "F.Cu") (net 9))
 (segment (start 33.0000 34.8000) (end 34.2000 36.0000) (width 0.2500) (layer "F.Cu") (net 9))
 (via (at 12.6000 22.2000) (size 0.6000) (drill 0.3000) (layers "F.Cu" "B.Cu") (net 2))
 (via (at 21.6000 27.6000) (size 0.6000) (drill 0.3000) (layers "F.Cu" "B.Cu") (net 8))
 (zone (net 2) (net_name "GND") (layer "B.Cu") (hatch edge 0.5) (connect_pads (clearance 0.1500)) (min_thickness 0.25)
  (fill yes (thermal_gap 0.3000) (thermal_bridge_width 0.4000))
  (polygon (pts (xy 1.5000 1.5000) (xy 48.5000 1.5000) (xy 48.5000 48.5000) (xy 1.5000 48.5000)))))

